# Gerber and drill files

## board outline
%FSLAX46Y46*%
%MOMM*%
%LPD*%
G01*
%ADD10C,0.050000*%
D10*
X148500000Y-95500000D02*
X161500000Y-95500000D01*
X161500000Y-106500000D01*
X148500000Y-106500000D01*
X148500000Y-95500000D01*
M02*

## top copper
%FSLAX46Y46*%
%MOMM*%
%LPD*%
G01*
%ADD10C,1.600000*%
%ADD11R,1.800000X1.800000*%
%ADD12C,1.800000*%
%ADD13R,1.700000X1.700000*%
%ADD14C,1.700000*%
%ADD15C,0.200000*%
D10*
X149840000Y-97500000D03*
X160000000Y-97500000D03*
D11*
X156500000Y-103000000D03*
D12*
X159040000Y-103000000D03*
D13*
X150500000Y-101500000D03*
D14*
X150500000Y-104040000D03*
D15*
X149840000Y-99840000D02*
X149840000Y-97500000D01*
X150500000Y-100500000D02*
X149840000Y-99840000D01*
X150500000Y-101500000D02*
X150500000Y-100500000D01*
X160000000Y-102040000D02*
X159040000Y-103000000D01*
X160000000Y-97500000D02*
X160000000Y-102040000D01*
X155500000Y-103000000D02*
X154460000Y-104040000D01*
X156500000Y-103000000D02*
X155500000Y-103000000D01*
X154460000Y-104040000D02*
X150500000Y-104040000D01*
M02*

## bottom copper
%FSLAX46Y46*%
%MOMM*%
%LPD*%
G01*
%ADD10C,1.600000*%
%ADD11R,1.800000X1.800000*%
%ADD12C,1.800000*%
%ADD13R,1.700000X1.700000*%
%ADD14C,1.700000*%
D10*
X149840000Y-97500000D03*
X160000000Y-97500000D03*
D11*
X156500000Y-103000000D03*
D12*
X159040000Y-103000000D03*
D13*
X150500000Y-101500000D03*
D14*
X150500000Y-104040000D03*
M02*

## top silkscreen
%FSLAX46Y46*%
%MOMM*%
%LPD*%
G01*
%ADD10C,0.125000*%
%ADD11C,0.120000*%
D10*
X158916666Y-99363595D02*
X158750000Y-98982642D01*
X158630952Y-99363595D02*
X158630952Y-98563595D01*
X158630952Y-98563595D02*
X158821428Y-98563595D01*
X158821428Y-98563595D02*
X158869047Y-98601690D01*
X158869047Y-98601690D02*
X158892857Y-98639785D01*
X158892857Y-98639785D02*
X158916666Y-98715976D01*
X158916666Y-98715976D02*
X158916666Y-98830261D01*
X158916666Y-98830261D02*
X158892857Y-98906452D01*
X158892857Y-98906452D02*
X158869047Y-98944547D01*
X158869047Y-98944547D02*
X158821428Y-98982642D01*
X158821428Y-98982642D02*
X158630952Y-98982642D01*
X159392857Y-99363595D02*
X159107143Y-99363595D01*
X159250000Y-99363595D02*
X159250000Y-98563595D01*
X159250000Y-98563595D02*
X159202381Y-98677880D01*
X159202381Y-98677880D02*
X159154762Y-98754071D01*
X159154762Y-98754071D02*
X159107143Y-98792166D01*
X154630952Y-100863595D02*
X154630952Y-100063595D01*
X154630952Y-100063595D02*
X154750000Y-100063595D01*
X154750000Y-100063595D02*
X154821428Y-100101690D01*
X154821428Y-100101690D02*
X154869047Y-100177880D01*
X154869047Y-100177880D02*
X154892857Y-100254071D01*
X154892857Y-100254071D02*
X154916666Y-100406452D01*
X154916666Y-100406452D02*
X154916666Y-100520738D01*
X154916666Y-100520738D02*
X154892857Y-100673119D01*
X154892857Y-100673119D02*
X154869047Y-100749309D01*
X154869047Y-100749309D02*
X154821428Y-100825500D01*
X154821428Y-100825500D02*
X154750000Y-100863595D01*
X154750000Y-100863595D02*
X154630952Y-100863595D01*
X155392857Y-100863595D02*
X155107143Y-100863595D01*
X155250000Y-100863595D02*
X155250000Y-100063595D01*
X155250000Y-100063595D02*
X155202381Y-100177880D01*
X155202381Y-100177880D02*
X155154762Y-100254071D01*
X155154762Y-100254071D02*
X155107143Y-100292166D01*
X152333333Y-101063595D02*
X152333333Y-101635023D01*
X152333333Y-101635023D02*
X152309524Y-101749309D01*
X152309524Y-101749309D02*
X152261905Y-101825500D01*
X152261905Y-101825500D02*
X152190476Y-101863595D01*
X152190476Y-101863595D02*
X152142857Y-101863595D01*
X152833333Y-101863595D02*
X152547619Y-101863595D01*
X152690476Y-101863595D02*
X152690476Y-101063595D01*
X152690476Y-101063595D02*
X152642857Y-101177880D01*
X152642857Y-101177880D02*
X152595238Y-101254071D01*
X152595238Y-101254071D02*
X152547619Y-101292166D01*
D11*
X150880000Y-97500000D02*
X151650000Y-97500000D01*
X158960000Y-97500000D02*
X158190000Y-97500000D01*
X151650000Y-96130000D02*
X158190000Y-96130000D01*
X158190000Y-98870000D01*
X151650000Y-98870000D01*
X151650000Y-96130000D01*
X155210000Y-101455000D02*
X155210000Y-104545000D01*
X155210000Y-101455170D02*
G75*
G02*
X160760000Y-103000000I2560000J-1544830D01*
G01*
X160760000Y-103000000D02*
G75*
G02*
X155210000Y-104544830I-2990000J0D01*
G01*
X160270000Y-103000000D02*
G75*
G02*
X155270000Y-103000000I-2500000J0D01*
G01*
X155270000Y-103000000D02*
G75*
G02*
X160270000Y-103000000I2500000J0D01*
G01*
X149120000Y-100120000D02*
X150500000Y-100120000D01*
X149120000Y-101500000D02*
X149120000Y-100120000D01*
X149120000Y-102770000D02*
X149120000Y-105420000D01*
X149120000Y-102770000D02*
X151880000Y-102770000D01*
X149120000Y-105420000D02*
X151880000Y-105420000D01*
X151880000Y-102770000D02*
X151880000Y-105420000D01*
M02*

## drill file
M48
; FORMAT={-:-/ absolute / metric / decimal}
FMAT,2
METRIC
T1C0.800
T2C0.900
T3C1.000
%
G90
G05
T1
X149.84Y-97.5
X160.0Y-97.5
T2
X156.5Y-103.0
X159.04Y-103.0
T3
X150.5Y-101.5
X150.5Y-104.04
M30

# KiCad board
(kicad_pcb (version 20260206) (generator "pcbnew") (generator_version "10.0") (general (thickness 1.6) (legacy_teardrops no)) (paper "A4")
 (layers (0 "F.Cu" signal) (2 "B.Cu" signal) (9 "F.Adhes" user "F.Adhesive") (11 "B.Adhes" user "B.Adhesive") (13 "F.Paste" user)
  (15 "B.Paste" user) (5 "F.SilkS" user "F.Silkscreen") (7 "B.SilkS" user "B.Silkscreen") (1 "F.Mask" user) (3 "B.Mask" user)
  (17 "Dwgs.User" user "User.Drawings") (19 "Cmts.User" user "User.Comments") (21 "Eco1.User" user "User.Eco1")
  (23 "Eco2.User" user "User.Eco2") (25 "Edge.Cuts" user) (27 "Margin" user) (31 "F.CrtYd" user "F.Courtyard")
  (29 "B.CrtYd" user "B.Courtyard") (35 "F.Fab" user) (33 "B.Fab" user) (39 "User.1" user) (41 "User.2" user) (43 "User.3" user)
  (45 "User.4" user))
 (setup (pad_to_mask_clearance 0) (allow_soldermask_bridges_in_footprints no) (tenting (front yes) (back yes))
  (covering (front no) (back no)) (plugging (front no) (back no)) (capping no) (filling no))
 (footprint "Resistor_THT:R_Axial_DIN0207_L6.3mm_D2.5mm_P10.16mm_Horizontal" (layer "F.Cu") (at 149.84 97.5)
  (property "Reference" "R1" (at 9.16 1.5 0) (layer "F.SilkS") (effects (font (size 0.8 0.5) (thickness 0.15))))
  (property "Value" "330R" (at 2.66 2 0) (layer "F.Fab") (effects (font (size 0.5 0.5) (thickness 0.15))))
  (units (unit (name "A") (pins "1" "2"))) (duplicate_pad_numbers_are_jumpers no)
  (fp_line (start 1.04 0) (end 1.81 0) (stroke (width 0.12) (type solid)) (layer "F.SilkS"))
  (fp_line (start 9.12 0) (end 8.35 0) (stroke (width 0.12) (type solid)) (layer "F.SilkS"))
  (fp_rect (start 1.81 -1.37) (end 8.35 1.37) (stroke (width 0.12) (type solid)) (fill no) (layer "F.SilkS"))
  (pad "1" thru_hole circle (at 0 0) (size 1.6 1.6) (drill 0.8) (layers "*.Cu" "*.Mask") (remove_unused_layers no) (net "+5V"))
  (pad "2" thru_hole circle (at 10.16 0) (size 1.6 1.6) (drill 0.8) (layers "*.Cu" "*.Mask") (remove_unused_layers no) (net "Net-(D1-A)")))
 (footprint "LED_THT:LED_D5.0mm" (layer "F.Cu") (at 156.5 103)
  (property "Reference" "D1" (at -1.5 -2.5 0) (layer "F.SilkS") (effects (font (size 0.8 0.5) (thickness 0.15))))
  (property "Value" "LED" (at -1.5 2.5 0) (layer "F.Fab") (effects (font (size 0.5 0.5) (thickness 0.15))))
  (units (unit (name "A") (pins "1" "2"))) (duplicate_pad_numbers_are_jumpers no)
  (fp_line (start -1.29 -1.545) (end -1.29 1.545) (stroke (width 0.12) (type solid)) (layer "F.SilkS"))
  (fp_arc (start -1.29 -1.54483) (mid 2.071779 -2.880495) (end 4.26 0) (stroke (width 0.12) (type solid)) (layer "F.SilkS"))
  (fp_arc (start 4.26 0) (mid 2.071779 2.880495) (end -1.29 1.54483) (stroke (width 0.12) (type solid)) (layer "F.SilkS"))
  (fp_circle (center 1.27 0) (end 3.77 0) (stroke (width 0.12) (type solid)) (fill no) (layer "F.SilkS"))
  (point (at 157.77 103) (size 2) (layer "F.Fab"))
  (pad "1" thru_hole rect (at 0 0) (size 1.8 1.8) (drill 0.9) (layers "*.Cu" "*.Mask") (remove_unused_layers no) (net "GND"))
  (pad "2" thru_hole circle (at 2.54 0) (size 1.8 1.8) (drill 0.9) (layers "*.Cu" "*.Mask") (remove_unused_layers no) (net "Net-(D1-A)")))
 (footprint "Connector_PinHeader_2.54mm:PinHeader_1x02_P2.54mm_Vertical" (layer "F.Cu") (at 150.5 101.5)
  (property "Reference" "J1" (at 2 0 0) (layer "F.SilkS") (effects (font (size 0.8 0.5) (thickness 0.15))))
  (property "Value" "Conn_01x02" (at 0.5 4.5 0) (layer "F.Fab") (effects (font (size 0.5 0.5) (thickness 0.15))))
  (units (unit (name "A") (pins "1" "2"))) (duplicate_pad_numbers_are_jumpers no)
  (fp_line (start -1.38 -1.38) (end 0 -1.38) (stroke (width 0.12) (type solid)) (layer "F.SilkS"))
  (fp_line (start -1.38 0) (end -1.38 -1.38) (stroke (width 0.12) (type solid)) (layer "F.SilkS"))
  (fp_line (start -1.38 1.27) (end -1.38 3.92) (stroke (width 0.12) (type solid)) (layer "F.SilkS"))
  (fp_line (start -1.38 1.27) (end 1.38 1.27) (stroke (width 0.12) (type solid)) (layer "F.SilkS"))
  (fp_line (start -1.38 3.92) (end 1.38 3.92) (stroke (width 0.12) (type solid)) (layer "F.SilkS"))
  (fp_line (start 1.38 1.27) (end 1.38 3.92) (stroke (width 0.12) (type solid)) (layer "F.SilkS"))
  (pad "1" thru_hole rect (at 0 0) (size 1.7 1.7) (drill 1) (layers "*.Cu" "*.Mask") (remove_unused_layers no) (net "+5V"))
  (pad "2" thru_hole circle (at 0 2.54) (size 1.7 1.7) (drill 1) (layers "*.Cu" "*.Mask") (remove_unused_layers no) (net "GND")))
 (gr_rect (start 148.5 95.5) (end 161.5 106.5) (stroke (width 0.05) (type default)) (fill no) (layer "Edge.Cuts"))
 (segment (start 149.84 99.84) (end 149.84 97.5) (width 0.2) (layer "F.Cu") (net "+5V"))
 (segment (start 150.5 100.5) (end 149.84 99.84) (width 0.2) (layer "F.Cu") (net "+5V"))
 (segment (start 150.5 101.5) (end 150.5 100.5) (width 0.2) (layer "F.Cu") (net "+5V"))
 (segment (start 160 102.04) (end 159.04 103) (width 0.2) (layer "F.Cu") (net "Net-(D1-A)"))
 (segment (start 160 97.5) (end 160 102.04) (width 0.2) (layer "F.Cu") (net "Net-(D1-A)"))
 (segment (start 155.5 103) (end 154.46 104.04) (width 0.2) (layer "F.Cu") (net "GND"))
 (segment (start 156.5 103) (end 155.5 103) (width 0.2) (layer "F.Cu") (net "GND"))
 (segment (start 154.46 104.04) (end 150.5 104.04) (width 0.2) (layer "F.Cu") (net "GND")))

